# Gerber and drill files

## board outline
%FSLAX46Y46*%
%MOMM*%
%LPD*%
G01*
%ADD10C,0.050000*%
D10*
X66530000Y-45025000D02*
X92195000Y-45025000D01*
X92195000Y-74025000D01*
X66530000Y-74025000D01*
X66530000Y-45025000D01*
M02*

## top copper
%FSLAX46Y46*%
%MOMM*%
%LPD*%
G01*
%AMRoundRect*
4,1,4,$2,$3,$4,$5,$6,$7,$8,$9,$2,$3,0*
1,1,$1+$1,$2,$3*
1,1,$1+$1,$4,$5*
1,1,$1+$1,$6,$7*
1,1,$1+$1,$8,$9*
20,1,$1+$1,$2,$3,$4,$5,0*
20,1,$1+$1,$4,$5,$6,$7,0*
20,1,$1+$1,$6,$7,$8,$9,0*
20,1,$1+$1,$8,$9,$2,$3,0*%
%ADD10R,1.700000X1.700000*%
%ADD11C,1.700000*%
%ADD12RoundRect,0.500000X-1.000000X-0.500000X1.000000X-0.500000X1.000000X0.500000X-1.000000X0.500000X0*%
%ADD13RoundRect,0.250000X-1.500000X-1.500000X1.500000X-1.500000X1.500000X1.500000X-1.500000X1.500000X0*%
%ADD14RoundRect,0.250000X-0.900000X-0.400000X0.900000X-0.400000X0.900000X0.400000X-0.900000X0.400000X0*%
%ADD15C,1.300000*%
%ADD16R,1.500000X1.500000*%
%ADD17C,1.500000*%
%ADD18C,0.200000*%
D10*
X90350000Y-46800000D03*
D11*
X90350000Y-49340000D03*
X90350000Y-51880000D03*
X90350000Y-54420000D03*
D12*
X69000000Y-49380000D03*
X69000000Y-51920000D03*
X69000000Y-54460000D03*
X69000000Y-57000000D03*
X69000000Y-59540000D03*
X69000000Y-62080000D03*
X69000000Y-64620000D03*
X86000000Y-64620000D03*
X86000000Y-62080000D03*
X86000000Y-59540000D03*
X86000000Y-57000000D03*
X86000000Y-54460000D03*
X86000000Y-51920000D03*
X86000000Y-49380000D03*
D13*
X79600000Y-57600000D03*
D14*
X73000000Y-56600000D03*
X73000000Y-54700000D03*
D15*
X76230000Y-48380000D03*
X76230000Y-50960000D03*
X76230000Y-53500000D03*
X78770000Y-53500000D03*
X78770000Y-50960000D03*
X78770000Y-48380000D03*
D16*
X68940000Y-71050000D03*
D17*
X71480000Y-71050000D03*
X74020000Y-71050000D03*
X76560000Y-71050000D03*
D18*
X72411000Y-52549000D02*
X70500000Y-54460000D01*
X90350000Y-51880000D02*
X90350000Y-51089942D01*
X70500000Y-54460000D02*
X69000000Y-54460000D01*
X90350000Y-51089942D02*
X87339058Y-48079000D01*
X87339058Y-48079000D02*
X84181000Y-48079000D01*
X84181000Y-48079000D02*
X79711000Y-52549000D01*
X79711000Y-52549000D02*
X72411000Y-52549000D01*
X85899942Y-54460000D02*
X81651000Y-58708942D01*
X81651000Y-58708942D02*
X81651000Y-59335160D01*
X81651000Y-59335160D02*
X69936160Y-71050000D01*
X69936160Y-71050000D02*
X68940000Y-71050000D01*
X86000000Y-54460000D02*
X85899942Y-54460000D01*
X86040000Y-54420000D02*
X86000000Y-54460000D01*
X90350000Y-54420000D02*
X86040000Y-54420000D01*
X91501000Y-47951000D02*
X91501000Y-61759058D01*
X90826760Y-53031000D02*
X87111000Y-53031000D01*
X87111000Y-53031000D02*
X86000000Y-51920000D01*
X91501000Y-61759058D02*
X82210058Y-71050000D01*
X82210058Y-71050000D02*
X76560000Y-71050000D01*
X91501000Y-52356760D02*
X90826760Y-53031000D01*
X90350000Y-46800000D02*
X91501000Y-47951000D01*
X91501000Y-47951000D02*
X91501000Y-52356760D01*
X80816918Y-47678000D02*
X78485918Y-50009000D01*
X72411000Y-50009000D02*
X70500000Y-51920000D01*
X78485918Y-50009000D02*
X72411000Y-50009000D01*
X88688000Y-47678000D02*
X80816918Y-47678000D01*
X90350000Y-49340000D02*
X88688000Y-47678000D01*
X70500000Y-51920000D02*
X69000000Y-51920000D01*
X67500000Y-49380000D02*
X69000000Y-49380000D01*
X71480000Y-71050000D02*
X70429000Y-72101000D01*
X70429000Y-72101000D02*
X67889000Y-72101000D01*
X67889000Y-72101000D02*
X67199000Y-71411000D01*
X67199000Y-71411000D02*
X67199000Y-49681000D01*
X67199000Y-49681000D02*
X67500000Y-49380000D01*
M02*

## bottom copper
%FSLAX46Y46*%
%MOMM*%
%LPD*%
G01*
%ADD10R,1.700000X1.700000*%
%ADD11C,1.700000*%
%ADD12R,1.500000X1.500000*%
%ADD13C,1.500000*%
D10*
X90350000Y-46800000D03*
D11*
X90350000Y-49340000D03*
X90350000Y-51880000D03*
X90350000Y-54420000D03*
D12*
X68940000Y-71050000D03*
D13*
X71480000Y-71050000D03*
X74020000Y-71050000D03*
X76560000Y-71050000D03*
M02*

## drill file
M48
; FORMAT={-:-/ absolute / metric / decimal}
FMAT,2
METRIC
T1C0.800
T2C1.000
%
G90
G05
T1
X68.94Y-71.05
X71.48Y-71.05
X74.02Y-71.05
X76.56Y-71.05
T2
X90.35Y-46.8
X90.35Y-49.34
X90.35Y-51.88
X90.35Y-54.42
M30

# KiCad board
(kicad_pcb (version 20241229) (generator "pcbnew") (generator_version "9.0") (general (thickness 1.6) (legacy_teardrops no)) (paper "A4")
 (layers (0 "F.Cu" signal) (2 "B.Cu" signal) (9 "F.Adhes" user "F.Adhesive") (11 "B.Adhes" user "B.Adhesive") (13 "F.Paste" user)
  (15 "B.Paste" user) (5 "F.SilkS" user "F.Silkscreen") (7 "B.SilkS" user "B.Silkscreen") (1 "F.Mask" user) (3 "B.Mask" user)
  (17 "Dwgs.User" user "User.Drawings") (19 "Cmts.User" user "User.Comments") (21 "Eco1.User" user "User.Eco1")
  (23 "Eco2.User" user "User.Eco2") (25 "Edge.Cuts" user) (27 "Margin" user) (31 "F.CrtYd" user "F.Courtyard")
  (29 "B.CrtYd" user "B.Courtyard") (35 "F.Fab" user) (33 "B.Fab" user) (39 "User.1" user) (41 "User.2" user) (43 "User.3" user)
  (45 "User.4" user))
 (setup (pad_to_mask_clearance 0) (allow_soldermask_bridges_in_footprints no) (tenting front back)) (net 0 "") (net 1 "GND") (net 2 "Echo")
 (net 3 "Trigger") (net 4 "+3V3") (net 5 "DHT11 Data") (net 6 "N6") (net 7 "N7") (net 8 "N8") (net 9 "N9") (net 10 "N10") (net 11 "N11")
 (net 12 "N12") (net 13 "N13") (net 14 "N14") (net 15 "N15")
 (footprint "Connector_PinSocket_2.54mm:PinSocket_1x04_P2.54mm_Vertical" (layer "F.Cu") (at 90.35 46.8)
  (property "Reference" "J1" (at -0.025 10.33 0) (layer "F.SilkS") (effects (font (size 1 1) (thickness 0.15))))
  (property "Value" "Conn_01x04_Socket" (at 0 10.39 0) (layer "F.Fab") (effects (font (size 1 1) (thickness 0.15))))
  (pad "1" thru_hole rect (at 0 0) (size 1.7 1.7) (drill 1) (layers "*.Cu" "*.Mask") (remove_unused_layers no) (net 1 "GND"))
  (pad "2" thru_hole circle (at 0 2.54) (size 1.7 1.7) (drill 1) (layers "*.Cu" "*.Mask") (remove_unused_layers no) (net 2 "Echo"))
  (pad "3" thru_hole circle (at 0 5.08) (size 1.7 1.7) (drill 1) (layers "*.Cu" "*.Mask") (remove_unused_layers no) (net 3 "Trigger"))
  (pad "4" thru_hole circle (at 0 7.62) (size 1.7 1.7) (drill 1) (layers "*.Cu" "*.Mask") (remove_unused_layers no) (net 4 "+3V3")))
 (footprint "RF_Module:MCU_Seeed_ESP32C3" (layer "F.Cu") (at 77.5 57)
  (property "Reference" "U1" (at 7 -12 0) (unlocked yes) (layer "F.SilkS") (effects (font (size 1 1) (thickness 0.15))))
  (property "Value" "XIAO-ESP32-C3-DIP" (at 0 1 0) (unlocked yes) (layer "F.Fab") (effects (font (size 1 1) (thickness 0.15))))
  (pad "" smd roundrect (at 1.1 -0.4) (size 1.5 1.5) (layers "F.Paste") (roundrect_rratio 0.1666666667))
  (pad "" smd roundrect (at 1.1 1.6) (size 1.5 1.5) (layers "F.Paste") (roundrect_rratio 0.1666666667))
  (pad "" smd roundrect (at 3.1 -0.4) (size 1.5 1.5) (layers "F.Paste") (roundrect_rratio 0.1666666667))
  (pad "" smd roundrect (at 3.1 1.6) (size 1.5 1.5) (layers "F.Paste") (roundrect_rratio 0.1666666667))
  (pad "1" smd roundrect (at -8.5 -7.62) (size 3 2) (layers "F.Cu" "F.Mask" "F.Paste") (roundrect_rratio 0.25) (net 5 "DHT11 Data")
   (thermal_bridge_angle 45))
  (pad "2" smd roundrect (at -8.5 -5.08) (size 3 2) (layers "F.Cu" "F.Mask" "F.Paste") (roundrect_rratio 0.25) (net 2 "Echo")
   (thermal_bridge_angle 45))
  (pad "3" smd roundrect (at -8.5 -2.54) (size 3 2) (layers "F.Cu" "F.Mask" "F.Paste") (roundrect_rratio 0.25) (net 3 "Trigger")
   (thermal_bridge_angle 45))
  (pad "4" smd roundrect (at -8.5 0) (size 3 2) (layers "F.Cu" "F.Mask" "F.Paste") (roundrect_rratio 0.25) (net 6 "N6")
   (thermal_bridge_angle 45))
  (pad "5" smd roundrect (at -8.5 2.54) (size 3 2) (layers "F.Cu" "F.Mask" "F.Paste") (roundrect_rratio 0.25) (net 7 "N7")
   (thermal_bridge_angle 45))
  (pad "6" smd roundrect (at -8.5 5.08) (size 3 2) (layers "F.Cu" "F.Mask" "F.Paste") (roundrect_rratio 0.25) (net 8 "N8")
   (thermal_bridge_angle 45))
  (pad "7" smd roundrect (at -8.5 7.62) (size 3 2) (layers "F.Cu" "F.Mask" "F.Paste") (roundrect_rratio 0.25) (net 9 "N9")
   (thermal_bridge_angle 45))
  (pad "8" smd roundrect (at 8.5 7.62) (size 3 2) (layers "F.Cu" "F.Mask" "F.Paste") (roundrect_rratio 0.25) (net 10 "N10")
   (thermal_bridge_angle 45))
  (pad "9" smd roundrect (at 8.5 5.08) (size 3 2) (layers "F.Cu" "F.Mask" "F.Paste") (roundrect_rratio 0.25) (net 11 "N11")
   (thermal_bridge_angle 45))
  (pad "10" smd roundrect (at 8.5 2.54) (size 3 2) (layers "F.Cu" "F.Mask" "F.Paste") (roundrect_rratio 0.25) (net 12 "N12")
   (thermal_bridge_angle 45))
  (pad "11" smd roundrect (at 8.5 0) (size 3 2) (layers "F.Cu" "F.Mask" "F.Paste") (roundrect_rratio 0.25) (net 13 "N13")
   (thermal_bridge_angle 45))
  (pad "12" smd roundrect (at 8.5 -2.54) (size 3 2) (layers "F.Cu" "F.Mask" "F.Paste") (roundrect_rratio 0.25) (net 4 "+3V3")
   (thermal_bridge_angle 45))
  (pad "13" smd roundrect (at 8.5 -5.08) (size 3 2) (layers "F.Cu" "F.Mask" "F.Paste") (roundrect_rratio 0.25) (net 1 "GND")
   (thermal_bridge_angle 45))
  (pad "14" smd roundrect (at 8.5 -7.62) (size 3 2) (layers "F.Cu" "F.Mask" "F.Paste") (roundrect_rratio 0.25) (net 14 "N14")
   (thermal_bridge_angle 45))
  (pad "15" smd roundrect (at 2.1 0.6) (size 3.5 3.5) (layers "F.Cu" "F.Mask") (roundrect_rratio 0.07142857143))
  (pad "16" smd roundrect (at -4.5 -0.4) (size 2.3 1.3) (layers "F.Cu" "F.Mask" "F.Paste") (roundrect_rratio 0.1923076923))
  (pad "17" smd roundrect (at -4.5 -2.3) (size 2.3 1.3) (layers "F.Cu" "F.Mask" "F.Paste") (roundrect_rratio 0.1923076923))
  (pad "18" smd circle (at -1.27 -8.62) (size 1.3 1.3) (layers "F.Cu" "F.Mask" "F.Paste"))
  (pad "19" smd circle (at -1.27 -6.04) (size 1.3 1.3) (layers "F.Cu" "F.Mask" "F.Paste"))
  (pad "20" smd circle (at -1.27 -3.5) (size 1.3 1.3) (layers "F.Cu" "F.Mask" "F.Paste"))
  (pad "21" smd circle (at 1.27 -3.5) (size 1.3 1.3) (layers "F.Cu" "F.Mask" "F.Paste"))
  (pad "22" smd circle (at 1.27 -6.04) (size 1.3 1.3) (layers "F.Cu" "F.Mask" "F.Paste"))
  (pad "23" smd circle (at 1.27 -8.62) (size 1.3 1.3) (layers "F.Cu" "F.Mask" "F.Paste")))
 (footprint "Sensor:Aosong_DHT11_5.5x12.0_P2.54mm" (layer "F.Cu") (at 68.94 71.05 90)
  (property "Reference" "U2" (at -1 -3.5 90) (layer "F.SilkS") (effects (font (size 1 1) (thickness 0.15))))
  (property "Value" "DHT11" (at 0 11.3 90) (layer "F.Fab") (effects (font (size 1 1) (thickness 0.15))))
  (pad "1" thru_hole rect (at 0 0 90) (size 1.5 1.5) (drill 0.8) (layers "*.Cu" "*.Mask") (remove_unused_layers no) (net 4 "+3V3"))
  (pad "2" thru_hole circle (at 0 2.54 90) (size 1.5 1.5) (drill 0.8) (layers "*.Cu" "*.Mask") (remove_unused_layers no)
   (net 5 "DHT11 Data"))
  (pad "3" thru_hole circle (at 0 5.08 90) (size 1.5 1.5) (drill 0.8) (layers "*.Cu" "*.Mask") (remove_unused_layers no) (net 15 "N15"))
  (pad "4" thru_hole circle (at 0 7.62 90) (size 1.5 1.5) (drill 0.8) (layers "*.Cu" "*.Mask") (remove_unused_layers no) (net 1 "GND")))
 (gr_rect (start 66.53 45.025) (end 92.195 74.025) (stroke (width 0.05) (type default)) (fill no) (layer "Edge.Cuts"))
 (segment (start 72.411 52.549) (end 70.5 54.46) (width 0.2) (layer "F.Cu") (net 3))
 (segment (start 90.35 51.88) (end 90.35 51.089942) (width 0.2) (layer "F.Cu") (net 3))
 (segment (start 70.5 54.46) (end 69 54.46) (width 0.2) (layer "F.Cu") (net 3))
 (segment (start 90.35 51.089942) (end 87.339058 48.079) (width 0.2) (layer "F.Cu") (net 3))
 (segment (start 87.339058 48.079) (end 84.181 48.079) (width 0.2) (layer "F.Cu") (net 3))
 (segment (start 84.181 48.079) (end 79.711 52.549) (width 0.2) (layer "F.Cu") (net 3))
 (segment (start 79.711 52.549) (end 72.411 52.549) (width 0.2) (layer "F.Cu") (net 3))
 (segment (start 85.899942 54.46) (end 81.651 58.708942) (width 0.2) (layer "F.Cu") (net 4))
 (segment (start 81.651 58.708942) (end 81.651 59.33516) (width 0.2) (layer "F.Cu") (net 4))
 (segment (start 81.651 59.33516) (end 69.93616 71.05) (width 0.2) (layer "F.Cu") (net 4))
 (segment (start 69.93616 71.05) (end 68.94 71.05) (width 0.2) (layer "F.Cu") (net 4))
 (segment (start 86 54.46) (end 85.899942 54.46) (width 0.2) (layer "F.Cu") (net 4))
 (segment (start 86.04 54.42) (end 86 54.46) (width 0.2) (layer "F.Cu") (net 4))
 (segment (start 90.35 54.42) (end 86.04 54.42) (width 0.2) (layer "F.Cu") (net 4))
 (segment (start 91.501 47.951) (end 91.501 61.759058) (width 0.2) (layer "F.Cu") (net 1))
 (segment (start 90.82676 53.031) (end 87.111 53.031) (width 0.2) (layer "F.Cu") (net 1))
 (segment (start 87.111 53.031) (end 86 51.92) (width 0.2) (layer "F.Cu") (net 1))
 (segment (start 91.501 61.759058) (end 82.210058 71.05) (width 0.2) (layer "F.Cu") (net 1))
 (segment (start 82.210058 71.05) (end 76.56 71.05) (width 0.2) (layer "F.Cu") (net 1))
 (segment (start 91.501 52.35676) (end 90.82676 53.031) (width 0.2) (layer "F.Cu") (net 1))
 (segment (start 90.35 46.8) (end 91.501 47.951) (width 0.2) (layer "F.Cu") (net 1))
 (segment (start 91.501 47.951) (end 91.501 52.35676) (width 0.2) (layer "F.Cu") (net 1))
 (segment (start 80.816918 47.678) (end 78.485918 50.009) (width 0.2) (layer "F.Cu") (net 2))
 (segment (start 72.411 50.009) (end 70.5 51.92) (width 0.2) (layer "F.Cu") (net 2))
 (segment (start 78.485918 50.009) (end 72.411 50.009) (width 0.2) (layer "F.Cu") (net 2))
 (segment (start 88.688 47.678) (end 80.816918 47.678) (width 0.2) (layer "F.Cu") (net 2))
 (segment (start 90.35 49.34) (end 88.688 47.678) (width 0.2) (layer "F.Cu") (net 2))
 (segment (start 70.5 51.92) (end 69 51.92) (width 0.2) (layer "F.Cu") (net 2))
 (segment (start 67.5 49.38) (end 69 49.38) (width 0.2) (layer "F.Cu") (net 5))
 (segment (start 71.48 71.05) (end 70.429 72.101) (width 0.2) (layer "F.Cu") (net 5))
 (segment (start 70.429 72.101) (end 67.889 72.101) (width 0.2) (layer "F.Cu") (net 5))
 (segment (start 67.889 72.101) (end 67.199 71.411) (width 0.2) (layer "F.Cu") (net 5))
 (segment (start 67.199 71.411) (end 67.199 49.681) (width 0.2) (layer "F.Cu") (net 5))
 (segment (start 67.199 49.681) (end 67.5 49.38) (width 0.2) (layer "F.Cu") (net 5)))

